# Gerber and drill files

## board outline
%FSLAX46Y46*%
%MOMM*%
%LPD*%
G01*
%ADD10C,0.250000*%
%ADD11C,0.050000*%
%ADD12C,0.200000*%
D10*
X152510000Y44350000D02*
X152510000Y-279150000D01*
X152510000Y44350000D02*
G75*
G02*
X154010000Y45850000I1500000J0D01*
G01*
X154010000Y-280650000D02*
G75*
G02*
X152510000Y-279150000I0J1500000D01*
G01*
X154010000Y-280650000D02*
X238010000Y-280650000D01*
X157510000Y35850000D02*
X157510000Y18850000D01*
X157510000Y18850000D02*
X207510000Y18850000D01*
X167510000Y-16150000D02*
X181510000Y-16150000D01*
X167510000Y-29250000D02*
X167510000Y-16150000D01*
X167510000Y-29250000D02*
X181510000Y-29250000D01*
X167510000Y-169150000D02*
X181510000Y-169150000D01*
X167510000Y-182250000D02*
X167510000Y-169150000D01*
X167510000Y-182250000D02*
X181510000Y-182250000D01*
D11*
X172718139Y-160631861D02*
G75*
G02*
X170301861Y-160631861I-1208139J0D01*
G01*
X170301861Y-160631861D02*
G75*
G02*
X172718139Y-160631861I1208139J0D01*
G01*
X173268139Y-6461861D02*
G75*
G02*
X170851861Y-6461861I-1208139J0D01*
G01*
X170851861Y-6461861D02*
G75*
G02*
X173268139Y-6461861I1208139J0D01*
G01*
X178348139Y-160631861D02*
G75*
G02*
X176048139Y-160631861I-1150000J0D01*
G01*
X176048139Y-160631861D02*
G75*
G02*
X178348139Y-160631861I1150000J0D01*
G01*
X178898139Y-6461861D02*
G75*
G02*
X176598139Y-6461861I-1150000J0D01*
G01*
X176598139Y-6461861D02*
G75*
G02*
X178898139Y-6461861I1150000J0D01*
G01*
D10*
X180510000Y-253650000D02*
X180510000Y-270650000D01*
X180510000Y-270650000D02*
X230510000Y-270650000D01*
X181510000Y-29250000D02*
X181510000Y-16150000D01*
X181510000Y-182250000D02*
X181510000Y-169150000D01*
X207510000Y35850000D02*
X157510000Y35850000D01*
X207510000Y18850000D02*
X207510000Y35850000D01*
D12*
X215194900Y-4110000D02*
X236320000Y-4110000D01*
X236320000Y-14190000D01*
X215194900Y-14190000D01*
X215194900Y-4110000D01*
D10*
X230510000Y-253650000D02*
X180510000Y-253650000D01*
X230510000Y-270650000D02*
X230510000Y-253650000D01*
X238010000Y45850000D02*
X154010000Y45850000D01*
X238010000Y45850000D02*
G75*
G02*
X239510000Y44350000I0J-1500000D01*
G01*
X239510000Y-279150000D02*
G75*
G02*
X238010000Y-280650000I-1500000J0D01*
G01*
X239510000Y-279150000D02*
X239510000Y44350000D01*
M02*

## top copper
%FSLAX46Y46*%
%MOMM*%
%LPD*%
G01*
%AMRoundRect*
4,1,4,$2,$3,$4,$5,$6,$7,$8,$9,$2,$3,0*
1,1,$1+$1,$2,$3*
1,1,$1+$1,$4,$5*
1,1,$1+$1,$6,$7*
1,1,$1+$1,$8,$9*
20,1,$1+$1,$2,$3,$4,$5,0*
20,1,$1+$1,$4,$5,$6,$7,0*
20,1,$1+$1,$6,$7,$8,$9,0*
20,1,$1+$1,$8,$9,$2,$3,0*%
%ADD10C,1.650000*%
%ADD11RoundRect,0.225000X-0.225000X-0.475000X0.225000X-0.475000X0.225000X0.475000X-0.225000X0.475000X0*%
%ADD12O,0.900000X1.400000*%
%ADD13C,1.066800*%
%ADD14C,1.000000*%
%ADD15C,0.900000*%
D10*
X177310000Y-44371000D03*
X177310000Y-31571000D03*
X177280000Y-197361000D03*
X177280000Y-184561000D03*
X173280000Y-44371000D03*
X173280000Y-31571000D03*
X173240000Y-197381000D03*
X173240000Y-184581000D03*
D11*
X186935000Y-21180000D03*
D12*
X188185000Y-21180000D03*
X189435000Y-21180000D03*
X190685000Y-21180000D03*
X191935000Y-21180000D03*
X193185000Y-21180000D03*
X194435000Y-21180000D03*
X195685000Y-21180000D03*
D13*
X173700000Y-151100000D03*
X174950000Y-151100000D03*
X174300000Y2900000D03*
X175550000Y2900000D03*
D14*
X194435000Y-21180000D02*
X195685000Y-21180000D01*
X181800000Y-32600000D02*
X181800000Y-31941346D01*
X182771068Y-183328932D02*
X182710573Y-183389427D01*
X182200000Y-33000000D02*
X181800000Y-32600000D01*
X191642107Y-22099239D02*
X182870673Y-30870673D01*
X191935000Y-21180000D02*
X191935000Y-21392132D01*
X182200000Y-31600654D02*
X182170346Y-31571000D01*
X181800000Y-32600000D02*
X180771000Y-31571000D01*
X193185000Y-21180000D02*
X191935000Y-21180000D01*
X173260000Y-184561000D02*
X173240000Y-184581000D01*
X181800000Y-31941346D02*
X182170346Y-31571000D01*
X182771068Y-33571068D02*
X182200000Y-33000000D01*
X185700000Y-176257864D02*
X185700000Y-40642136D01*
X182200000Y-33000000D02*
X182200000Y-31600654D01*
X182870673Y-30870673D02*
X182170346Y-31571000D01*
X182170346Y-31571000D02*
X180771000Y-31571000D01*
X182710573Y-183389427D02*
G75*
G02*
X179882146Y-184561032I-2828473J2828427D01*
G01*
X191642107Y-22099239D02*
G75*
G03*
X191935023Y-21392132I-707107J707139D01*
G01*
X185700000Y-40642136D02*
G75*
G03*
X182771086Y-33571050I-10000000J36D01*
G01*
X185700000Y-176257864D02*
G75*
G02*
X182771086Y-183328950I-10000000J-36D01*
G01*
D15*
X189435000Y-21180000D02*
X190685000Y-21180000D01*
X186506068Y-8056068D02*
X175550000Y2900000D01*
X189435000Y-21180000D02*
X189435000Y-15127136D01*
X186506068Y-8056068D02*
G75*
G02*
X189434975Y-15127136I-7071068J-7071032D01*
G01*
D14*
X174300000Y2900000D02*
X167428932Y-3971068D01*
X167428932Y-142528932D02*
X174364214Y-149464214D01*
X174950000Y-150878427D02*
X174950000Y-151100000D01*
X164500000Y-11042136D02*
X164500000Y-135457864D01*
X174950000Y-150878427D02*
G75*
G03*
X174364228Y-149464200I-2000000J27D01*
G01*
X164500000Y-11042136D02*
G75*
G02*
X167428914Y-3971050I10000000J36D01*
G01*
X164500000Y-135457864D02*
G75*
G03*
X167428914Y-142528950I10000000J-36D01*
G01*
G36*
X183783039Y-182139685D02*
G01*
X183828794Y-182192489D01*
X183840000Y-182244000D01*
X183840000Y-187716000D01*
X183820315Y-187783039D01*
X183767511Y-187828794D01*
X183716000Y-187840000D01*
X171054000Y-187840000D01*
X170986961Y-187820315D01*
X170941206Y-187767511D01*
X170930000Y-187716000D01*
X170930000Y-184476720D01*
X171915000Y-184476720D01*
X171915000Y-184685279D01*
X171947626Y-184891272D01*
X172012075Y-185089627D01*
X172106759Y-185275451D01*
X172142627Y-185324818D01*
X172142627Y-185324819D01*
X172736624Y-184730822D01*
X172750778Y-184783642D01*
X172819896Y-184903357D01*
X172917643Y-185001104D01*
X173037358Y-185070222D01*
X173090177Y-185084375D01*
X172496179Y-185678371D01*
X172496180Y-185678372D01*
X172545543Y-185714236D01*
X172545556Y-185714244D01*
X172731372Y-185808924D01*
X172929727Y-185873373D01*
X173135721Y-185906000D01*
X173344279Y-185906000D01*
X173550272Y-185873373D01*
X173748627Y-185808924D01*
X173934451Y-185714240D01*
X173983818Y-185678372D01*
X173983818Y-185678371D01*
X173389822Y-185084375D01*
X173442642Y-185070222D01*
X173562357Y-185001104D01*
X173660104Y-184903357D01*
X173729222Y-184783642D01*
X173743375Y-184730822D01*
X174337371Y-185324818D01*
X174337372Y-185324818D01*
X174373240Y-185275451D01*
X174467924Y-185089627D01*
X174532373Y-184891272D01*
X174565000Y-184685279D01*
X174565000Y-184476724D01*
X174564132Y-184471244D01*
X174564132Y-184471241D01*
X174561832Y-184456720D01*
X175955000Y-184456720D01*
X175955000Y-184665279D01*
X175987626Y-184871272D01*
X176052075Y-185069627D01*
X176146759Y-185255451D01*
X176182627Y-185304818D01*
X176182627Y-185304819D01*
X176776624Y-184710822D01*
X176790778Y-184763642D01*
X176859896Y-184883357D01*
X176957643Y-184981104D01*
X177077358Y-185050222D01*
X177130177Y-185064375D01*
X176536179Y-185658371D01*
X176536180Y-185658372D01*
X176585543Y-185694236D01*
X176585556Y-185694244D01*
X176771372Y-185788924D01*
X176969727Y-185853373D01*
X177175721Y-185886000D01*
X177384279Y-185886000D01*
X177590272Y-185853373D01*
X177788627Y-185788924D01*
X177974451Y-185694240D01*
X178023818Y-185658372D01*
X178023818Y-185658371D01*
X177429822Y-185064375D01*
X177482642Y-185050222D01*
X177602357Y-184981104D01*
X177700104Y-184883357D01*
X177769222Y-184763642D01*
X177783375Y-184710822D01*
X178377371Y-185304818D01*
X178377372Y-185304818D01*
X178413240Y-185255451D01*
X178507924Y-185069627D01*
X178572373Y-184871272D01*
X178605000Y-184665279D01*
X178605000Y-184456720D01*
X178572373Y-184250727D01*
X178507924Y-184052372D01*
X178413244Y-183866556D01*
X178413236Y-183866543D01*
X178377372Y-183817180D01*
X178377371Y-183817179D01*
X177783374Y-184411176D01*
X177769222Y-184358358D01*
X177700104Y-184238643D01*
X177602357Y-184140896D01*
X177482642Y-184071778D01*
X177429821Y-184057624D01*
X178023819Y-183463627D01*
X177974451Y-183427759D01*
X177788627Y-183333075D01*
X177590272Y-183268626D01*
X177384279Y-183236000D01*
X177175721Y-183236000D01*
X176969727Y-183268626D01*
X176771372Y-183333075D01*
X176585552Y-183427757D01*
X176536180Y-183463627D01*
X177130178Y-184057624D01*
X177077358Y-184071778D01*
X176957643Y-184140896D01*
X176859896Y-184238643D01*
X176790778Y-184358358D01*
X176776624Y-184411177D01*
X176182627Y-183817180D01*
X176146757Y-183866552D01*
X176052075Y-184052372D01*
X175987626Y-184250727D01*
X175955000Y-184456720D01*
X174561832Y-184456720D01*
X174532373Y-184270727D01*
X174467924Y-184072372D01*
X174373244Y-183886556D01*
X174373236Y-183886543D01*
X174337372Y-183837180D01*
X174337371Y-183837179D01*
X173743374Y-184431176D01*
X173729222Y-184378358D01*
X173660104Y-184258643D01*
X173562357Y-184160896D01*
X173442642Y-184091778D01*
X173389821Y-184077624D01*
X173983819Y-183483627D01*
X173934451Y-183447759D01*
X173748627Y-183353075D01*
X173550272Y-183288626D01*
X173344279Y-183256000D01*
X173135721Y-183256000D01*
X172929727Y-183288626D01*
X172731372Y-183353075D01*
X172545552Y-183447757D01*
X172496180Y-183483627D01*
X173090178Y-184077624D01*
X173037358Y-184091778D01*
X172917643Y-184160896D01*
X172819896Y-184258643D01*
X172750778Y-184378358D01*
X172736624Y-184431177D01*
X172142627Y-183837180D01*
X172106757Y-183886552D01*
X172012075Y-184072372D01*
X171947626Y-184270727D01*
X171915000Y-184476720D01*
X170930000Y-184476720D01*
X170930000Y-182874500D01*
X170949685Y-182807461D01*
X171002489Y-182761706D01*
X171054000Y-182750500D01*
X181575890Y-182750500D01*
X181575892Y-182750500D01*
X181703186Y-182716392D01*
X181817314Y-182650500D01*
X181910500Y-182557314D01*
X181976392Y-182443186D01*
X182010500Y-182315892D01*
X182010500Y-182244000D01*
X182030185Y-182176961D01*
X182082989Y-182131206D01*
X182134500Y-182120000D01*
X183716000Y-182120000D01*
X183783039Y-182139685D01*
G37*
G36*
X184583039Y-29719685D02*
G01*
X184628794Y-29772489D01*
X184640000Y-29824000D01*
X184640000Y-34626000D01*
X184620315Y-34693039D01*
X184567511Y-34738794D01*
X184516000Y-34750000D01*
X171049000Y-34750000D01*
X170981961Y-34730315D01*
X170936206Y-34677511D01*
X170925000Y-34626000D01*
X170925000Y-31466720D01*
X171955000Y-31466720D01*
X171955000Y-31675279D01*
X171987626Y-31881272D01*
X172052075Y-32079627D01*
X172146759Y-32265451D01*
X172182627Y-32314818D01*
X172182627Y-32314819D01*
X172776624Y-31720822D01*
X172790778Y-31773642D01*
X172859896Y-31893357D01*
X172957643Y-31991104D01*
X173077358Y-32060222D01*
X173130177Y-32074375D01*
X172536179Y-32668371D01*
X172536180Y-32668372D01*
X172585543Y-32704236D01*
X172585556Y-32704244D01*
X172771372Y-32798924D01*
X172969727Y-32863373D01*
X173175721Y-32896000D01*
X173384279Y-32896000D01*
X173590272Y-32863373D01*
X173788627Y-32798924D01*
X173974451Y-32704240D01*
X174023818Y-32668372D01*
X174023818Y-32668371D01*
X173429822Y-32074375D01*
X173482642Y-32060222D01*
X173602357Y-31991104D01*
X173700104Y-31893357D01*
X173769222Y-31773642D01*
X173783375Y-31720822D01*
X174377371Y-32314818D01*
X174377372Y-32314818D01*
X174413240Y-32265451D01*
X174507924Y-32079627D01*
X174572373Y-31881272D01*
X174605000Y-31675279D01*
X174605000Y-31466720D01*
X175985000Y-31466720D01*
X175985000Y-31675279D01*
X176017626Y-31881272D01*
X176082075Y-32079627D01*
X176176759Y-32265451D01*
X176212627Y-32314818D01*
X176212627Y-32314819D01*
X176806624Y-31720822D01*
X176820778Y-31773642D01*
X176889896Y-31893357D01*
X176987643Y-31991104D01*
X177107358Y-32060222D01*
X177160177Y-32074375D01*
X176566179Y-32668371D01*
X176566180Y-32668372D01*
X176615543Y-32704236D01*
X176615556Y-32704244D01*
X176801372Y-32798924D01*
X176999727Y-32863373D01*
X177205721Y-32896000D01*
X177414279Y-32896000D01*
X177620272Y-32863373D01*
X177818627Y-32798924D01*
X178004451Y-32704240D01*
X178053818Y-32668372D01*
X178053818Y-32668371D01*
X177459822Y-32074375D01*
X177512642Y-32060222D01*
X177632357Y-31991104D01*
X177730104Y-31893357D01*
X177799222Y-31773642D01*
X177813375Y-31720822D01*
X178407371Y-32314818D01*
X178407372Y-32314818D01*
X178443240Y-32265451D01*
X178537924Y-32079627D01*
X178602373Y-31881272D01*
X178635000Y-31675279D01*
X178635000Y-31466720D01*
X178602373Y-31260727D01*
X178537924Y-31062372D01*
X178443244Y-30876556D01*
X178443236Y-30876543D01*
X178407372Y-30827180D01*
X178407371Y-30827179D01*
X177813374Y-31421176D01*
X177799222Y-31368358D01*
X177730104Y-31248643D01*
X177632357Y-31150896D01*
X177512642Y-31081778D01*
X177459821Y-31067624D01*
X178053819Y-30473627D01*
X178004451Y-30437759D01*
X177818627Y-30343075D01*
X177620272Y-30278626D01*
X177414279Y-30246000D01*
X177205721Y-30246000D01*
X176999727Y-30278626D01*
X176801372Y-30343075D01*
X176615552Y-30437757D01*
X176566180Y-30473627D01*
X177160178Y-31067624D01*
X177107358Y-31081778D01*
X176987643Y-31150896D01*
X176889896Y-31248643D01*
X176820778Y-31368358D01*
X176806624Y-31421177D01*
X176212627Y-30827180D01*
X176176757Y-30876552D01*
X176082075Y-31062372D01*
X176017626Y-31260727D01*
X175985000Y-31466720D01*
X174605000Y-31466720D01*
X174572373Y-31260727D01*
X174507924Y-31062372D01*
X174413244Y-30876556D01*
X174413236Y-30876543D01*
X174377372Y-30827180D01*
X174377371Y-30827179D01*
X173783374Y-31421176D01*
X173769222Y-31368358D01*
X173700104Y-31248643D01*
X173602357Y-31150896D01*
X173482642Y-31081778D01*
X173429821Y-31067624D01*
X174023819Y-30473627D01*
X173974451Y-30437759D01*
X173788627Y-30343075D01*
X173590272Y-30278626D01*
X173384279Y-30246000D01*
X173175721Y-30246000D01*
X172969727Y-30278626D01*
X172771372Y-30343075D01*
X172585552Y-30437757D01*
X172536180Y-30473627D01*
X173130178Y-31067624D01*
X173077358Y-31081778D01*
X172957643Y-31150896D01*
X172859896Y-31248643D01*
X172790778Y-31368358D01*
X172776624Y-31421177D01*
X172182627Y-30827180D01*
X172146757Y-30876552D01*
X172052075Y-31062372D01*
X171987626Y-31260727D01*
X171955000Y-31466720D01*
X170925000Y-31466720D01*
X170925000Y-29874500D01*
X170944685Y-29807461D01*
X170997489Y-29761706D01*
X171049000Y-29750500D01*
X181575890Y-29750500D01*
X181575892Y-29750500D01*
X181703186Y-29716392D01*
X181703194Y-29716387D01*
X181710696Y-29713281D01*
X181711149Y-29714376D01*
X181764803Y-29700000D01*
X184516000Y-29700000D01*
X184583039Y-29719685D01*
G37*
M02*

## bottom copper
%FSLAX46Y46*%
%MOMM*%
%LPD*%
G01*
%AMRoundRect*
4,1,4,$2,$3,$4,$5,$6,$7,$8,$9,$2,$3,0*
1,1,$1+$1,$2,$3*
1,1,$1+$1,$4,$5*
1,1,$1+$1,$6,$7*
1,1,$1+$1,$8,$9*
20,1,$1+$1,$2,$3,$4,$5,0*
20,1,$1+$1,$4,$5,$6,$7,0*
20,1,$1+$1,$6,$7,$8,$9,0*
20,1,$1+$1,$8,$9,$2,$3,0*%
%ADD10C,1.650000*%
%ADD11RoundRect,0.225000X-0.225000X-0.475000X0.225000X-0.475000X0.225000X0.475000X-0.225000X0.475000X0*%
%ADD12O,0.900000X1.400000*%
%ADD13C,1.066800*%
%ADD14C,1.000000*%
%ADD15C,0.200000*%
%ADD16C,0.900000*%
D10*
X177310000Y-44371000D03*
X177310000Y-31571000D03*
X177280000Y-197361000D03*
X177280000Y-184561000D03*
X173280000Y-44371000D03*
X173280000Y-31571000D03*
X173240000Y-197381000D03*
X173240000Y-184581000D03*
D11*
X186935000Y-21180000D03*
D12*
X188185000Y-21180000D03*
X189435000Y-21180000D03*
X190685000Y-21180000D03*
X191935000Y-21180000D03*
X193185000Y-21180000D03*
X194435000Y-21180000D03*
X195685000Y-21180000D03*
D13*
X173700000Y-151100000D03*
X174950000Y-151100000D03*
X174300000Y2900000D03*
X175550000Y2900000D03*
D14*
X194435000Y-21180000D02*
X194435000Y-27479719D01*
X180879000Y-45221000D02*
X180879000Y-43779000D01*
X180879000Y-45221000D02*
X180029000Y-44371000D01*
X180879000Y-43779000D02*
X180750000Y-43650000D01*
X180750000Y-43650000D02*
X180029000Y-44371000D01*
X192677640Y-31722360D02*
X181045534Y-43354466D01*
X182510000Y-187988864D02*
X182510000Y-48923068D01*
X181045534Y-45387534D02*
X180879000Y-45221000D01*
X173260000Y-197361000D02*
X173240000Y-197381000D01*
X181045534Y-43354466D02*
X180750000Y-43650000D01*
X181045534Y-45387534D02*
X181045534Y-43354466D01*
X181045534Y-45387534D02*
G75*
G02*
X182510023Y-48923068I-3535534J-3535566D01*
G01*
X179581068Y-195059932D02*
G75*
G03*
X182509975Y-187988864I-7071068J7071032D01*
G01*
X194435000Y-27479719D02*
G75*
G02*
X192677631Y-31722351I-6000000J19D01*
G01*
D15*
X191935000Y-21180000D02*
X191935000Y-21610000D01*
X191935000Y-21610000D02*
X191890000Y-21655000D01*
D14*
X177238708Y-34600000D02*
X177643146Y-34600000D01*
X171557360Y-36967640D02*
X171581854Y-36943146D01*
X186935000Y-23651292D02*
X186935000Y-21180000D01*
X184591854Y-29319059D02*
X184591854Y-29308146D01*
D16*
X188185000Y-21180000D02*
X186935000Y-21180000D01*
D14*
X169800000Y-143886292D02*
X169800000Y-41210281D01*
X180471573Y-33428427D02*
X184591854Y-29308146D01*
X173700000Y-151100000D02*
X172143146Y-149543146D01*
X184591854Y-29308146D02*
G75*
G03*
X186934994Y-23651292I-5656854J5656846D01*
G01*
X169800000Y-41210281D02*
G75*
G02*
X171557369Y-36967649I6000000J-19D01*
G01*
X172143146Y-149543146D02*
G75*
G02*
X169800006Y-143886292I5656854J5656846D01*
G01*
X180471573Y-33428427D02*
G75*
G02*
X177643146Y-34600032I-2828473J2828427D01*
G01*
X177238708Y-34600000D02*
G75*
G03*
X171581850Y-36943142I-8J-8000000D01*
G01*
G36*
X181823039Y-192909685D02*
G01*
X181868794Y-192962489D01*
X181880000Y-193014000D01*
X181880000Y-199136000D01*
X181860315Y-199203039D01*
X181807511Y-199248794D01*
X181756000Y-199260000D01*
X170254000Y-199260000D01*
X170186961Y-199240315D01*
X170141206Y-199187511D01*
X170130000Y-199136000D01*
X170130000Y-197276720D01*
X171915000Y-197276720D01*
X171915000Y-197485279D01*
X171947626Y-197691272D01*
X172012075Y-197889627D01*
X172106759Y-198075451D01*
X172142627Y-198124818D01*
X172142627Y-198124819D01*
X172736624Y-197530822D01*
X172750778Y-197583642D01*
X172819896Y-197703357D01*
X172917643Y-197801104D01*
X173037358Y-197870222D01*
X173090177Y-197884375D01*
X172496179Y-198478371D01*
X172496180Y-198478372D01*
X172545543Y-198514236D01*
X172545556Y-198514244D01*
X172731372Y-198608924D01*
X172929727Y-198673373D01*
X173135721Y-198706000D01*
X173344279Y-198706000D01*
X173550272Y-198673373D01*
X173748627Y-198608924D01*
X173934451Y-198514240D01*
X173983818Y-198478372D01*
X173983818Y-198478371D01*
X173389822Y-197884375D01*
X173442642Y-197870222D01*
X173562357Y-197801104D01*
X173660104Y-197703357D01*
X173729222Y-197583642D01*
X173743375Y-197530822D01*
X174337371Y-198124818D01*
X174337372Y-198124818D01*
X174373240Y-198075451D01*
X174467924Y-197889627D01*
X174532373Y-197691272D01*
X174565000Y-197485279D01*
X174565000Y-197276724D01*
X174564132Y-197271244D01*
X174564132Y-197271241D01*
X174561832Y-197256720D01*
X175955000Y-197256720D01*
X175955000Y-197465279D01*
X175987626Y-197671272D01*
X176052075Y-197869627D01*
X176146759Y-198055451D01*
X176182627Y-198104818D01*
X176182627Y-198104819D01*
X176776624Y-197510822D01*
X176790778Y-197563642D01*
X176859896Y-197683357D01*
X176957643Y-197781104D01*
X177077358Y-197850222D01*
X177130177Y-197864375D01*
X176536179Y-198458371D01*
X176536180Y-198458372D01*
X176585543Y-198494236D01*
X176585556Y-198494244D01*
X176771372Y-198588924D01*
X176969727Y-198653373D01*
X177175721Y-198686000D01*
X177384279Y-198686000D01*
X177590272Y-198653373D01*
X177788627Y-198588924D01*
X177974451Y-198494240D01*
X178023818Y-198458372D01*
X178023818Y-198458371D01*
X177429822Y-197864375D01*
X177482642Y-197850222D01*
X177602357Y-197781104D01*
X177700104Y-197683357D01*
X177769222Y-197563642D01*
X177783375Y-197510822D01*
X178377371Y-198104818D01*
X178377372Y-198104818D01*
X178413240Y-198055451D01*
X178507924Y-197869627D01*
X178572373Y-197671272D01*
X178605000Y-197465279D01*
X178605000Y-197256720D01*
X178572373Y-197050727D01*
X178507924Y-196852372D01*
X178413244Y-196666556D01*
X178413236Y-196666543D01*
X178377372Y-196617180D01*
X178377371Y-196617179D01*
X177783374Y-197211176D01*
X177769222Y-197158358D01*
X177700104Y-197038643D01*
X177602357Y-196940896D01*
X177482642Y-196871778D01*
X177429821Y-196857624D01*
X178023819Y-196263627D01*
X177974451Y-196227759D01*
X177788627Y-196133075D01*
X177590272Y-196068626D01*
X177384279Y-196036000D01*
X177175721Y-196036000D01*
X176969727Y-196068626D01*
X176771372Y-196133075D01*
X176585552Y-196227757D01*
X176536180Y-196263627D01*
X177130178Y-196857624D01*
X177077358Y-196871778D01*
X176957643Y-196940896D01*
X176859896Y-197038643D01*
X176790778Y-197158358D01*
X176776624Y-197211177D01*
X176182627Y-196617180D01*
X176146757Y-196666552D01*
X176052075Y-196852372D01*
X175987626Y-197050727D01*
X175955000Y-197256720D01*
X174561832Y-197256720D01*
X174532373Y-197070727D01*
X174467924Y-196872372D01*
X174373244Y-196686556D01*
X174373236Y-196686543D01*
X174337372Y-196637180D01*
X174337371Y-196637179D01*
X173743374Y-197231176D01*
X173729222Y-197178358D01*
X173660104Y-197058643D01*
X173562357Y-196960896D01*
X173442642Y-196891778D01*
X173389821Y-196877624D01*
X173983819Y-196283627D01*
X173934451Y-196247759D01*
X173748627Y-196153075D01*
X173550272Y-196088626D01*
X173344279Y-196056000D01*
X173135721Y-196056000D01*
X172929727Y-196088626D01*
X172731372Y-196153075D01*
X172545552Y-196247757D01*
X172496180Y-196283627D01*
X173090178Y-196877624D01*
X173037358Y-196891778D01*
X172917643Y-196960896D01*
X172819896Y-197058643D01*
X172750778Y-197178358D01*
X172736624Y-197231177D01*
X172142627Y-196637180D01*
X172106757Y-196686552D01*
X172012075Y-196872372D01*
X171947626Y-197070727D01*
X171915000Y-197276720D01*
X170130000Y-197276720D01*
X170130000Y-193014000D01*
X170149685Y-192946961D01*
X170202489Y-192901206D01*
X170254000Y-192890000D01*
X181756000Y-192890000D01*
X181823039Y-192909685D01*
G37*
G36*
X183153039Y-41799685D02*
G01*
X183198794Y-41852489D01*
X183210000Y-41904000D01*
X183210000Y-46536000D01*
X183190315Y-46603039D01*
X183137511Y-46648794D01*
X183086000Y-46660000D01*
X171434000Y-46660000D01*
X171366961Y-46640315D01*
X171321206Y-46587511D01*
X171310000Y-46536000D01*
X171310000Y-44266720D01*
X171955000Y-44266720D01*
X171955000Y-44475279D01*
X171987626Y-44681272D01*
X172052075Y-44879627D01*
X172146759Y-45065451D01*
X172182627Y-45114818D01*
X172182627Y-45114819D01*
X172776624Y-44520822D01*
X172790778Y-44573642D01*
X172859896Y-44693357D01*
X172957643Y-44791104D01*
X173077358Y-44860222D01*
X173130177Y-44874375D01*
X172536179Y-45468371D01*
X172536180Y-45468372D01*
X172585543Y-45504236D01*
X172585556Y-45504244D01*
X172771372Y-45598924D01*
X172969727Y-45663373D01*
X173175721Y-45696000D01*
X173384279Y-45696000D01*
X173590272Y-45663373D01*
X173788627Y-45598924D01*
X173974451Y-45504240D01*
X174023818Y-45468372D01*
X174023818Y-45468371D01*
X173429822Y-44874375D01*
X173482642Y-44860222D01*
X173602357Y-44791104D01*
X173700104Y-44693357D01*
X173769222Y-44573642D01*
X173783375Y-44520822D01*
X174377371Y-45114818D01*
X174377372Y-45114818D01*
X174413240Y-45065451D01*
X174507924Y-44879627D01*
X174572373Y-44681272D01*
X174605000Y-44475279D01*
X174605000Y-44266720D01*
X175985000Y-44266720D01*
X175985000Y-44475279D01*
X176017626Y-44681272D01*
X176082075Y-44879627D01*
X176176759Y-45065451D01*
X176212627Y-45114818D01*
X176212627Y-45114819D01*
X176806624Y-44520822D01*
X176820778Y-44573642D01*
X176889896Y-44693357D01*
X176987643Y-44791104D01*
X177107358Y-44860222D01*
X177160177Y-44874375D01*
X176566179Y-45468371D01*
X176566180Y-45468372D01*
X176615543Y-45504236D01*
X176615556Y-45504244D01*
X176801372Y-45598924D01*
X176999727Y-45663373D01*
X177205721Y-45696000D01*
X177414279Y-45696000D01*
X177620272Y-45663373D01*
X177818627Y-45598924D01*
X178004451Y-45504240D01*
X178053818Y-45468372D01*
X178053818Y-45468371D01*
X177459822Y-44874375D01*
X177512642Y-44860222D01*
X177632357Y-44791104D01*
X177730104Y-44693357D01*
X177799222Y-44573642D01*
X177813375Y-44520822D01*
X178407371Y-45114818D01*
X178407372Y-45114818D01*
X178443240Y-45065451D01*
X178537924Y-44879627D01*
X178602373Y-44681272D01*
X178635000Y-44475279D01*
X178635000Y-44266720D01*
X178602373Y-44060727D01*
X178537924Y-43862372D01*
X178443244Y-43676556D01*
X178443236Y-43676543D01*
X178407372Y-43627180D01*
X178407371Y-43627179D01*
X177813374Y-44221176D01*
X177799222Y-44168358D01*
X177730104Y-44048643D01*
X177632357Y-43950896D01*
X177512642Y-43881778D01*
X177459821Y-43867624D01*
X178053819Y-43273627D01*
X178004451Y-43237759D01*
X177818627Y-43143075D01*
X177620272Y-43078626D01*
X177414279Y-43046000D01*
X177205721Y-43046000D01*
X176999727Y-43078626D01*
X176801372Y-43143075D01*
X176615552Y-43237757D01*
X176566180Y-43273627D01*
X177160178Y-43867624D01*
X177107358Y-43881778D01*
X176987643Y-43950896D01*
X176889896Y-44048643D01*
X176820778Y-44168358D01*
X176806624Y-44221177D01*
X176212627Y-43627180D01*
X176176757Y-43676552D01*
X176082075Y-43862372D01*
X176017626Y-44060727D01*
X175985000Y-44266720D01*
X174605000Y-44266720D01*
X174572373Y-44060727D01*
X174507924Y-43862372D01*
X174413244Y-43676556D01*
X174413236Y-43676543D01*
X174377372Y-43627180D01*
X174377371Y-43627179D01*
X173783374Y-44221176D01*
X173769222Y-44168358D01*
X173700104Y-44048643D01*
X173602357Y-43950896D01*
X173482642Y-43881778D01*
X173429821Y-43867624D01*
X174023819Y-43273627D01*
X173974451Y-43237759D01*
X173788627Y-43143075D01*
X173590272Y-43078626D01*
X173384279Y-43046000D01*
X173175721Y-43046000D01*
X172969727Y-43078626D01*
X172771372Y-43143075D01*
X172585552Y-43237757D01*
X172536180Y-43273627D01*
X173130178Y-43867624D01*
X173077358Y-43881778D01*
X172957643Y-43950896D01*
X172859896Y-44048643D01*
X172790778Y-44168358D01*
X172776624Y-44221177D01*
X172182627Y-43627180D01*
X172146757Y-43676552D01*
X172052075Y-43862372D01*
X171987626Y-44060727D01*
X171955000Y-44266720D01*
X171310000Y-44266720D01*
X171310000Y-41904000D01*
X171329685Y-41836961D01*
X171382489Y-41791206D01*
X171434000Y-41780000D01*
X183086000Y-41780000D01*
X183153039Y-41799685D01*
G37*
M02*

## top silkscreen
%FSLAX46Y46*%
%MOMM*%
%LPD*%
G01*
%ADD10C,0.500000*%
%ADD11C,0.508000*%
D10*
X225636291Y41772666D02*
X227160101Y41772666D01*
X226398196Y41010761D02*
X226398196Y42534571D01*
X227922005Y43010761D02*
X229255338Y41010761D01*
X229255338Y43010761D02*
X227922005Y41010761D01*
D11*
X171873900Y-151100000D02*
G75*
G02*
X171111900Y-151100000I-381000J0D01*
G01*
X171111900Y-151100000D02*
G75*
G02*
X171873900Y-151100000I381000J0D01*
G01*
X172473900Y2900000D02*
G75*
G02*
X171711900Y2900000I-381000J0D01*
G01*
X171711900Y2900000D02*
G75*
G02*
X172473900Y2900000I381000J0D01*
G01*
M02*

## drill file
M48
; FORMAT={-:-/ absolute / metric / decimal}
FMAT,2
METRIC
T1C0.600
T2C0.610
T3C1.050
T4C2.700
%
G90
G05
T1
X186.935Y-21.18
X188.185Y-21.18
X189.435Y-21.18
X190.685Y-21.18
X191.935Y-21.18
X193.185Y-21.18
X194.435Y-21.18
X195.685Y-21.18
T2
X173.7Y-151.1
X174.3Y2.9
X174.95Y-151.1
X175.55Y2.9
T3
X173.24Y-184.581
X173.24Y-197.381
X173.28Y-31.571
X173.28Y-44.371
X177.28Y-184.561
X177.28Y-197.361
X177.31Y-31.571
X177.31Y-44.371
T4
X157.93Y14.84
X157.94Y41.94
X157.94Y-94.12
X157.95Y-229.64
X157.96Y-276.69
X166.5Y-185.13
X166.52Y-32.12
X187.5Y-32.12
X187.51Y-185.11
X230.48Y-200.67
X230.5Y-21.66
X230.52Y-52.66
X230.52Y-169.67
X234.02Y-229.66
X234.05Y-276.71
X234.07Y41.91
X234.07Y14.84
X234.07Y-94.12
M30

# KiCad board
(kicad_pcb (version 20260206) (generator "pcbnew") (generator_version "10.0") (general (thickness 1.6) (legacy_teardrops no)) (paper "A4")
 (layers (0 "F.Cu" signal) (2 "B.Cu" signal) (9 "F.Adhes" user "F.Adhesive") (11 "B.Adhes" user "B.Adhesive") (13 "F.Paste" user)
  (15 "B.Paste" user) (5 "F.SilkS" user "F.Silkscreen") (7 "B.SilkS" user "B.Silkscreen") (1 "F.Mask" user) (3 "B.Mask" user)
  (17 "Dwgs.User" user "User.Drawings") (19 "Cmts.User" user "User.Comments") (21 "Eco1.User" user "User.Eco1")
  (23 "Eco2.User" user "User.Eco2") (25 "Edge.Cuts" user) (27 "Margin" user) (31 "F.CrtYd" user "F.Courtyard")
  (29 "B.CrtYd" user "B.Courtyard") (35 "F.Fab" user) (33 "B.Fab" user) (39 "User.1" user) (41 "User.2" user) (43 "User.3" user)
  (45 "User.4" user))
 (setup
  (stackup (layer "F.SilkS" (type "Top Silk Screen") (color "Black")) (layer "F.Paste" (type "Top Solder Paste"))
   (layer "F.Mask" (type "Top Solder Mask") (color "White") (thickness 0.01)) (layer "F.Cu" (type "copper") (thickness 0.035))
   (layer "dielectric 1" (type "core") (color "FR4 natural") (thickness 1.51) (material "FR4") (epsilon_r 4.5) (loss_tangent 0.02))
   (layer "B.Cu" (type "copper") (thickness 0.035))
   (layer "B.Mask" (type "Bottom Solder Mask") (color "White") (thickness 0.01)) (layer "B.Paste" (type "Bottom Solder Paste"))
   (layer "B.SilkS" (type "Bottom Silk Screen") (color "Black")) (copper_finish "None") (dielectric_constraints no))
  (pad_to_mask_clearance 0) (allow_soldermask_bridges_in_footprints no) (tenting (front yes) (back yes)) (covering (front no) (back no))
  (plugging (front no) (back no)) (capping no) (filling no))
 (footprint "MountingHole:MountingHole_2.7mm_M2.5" (layer "F.Cu") (at 230.52 169.67 180)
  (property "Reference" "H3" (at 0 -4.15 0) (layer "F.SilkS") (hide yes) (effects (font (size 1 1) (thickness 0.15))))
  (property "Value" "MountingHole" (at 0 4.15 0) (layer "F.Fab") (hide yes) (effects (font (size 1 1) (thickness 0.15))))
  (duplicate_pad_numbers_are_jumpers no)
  (pad "" np_thru_hole circle (at 0 0 180) (size 2.7 2.7) (drill 2.7) (layers "*.Cu" "*.Mask")))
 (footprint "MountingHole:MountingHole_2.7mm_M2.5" (layer "F.Cu") (at 187.5 32.12)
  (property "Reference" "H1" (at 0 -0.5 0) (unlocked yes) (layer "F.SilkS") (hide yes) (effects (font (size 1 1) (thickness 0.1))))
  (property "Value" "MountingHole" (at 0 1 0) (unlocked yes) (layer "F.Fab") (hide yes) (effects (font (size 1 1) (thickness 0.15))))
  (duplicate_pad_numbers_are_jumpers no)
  (pad "" np_thru_hole circle (at 0 0) (size 2.7 2.7) (drill 2.7) (layers "*.Cu" "*.Mask")))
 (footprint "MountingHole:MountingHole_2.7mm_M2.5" (layer "F.Cu") (at 234.07 -41.91 180)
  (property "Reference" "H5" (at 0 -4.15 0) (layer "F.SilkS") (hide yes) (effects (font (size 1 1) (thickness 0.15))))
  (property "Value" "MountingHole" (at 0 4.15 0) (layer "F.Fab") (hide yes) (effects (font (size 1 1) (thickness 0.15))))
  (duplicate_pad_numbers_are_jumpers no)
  (pad "" np_thru_hole circle (at 0 0 180) (size 2.7 2.7) (drill 2.7) (layers "*.Cu" "*.Mask")))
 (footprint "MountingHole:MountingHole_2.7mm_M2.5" (layer "F.Cu") (at 230.48 200.67 180)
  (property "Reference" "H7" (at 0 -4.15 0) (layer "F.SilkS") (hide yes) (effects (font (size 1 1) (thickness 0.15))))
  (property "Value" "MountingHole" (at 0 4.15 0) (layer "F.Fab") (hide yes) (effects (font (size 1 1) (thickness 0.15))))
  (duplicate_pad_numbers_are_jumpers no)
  (pad "" np_thru_hole circle (at 0 0 180) (size 2.7 2.7) (drill 2.7) (layers "*.Cu" "*.Mask")))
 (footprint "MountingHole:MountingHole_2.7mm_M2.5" (layer "F.Cu") (at 157.94 -41.94 180)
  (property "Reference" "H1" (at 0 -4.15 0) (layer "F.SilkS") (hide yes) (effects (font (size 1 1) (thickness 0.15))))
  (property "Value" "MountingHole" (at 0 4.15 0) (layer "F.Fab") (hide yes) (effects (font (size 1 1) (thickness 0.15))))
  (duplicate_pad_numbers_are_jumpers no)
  (pad "" np_thru_hole circle (at 0 0 180) (size 2.7 2.7) (drill 2.7) (layers "*.Cu" "*.Mask")))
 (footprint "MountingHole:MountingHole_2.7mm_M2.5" (layer "F.Cu") (at 166.5 185.13)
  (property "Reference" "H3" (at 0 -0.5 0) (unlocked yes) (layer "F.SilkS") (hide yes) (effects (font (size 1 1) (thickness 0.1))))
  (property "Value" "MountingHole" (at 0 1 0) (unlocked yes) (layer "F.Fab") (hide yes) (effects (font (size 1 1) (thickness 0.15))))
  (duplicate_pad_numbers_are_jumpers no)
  (pad "" np_thru_hole circle (at 0 0) (size 2.7 2.7) (drill 2.7) (layers "*.Cu" "*.Mask")))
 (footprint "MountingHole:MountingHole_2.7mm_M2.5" (layer "F.Cu") (at 234.05 276.71 180)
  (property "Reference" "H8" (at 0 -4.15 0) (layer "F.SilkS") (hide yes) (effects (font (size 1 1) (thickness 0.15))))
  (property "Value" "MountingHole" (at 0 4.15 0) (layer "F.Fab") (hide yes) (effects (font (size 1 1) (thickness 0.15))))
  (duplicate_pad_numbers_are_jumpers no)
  (pad "" np_thru_hole circle (at 0 0 180) (size 2.7 2.7) (drill 2.7) (layers "*.Cu" "*.Mask")))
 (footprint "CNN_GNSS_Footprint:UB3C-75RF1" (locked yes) (layer "F.Cu") (at 177.31 44.371 90)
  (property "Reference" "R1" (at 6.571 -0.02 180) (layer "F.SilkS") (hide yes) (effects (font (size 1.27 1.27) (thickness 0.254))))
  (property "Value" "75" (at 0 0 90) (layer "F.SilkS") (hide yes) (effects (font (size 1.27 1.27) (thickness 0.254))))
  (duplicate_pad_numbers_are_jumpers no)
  (pad "1" thru_hole circle (at 0 0 90) (size 1.65 1.65) (drill 1.05) (layers "*.Cu" "*.Mask") (remove_unused_layers no) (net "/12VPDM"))
  (pad "2" thru_hole circle (at 12.8 0 90) (size 1.65 1.65) (drill 1.05) (layers "*.Cu" "*.Mask") (remove_unused_layers no)
   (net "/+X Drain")))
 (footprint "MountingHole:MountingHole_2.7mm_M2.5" (layer "F.Cu") (at 230.52 52.66 180)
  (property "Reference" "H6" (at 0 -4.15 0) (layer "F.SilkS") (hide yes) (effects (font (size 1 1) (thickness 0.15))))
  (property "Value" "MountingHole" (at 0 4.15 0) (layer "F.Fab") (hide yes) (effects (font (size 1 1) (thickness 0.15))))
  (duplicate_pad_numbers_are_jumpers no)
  (pad "" np_thru_hole circle (at 0 0 180) (size 2.7 2.7) (drill 2.7) (layers "*.Cu" "*.Mask")))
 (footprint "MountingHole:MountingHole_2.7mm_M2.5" (layer "F.Cu") (at 166.52 32.12)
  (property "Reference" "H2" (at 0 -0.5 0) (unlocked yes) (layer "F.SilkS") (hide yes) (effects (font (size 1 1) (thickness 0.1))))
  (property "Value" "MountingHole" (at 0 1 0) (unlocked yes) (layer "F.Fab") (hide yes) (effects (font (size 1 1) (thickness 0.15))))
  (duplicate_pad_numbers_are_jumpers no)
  (pad "" np_thru_hole circle (at 0 0) (size 2.7 2.7) (drill 2.7) (layers "*.Cu" "*.Mask")))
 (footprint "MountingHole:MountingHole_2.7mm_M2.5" (layer "F.Cu") (at 234.07 -14.84 180)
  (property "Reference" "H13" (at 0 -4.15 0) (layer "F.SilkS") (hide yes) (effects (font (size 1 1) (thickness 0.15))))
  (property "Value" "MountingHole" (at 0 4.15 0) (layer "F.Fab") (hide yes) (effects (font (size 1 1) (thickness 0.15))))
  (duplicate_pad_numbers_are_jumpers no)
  (pad "" np_thru_hole circle (at 0 0 180) (size 2.7 2.7) (drill 2.7) (layers "*.Cu" "*.Mask")))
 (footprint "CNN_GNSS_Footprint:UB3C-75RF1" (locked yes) (layer "F.Cu") (at 177.28 197.361 90)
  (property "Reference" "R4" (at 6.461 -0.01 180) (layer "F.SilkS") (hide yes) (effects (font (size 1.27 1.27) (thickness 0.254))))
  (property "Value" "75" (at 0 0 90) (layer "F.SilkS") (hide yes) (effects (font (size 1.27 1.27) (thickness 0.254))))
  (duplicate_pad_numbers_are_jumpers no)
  (pad "1" thru_hole circle (at 0 0 90) (size 1.65 1.65) (drill 1.05) (layers "*.Cu" "*.Mask") (remove_unused_layers no) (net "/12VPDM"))
  (pad "2" thru_hole circle (at 12.8 0 90) (size 1.65 1.65) (drill 1.05) (layers "*.Cu" "*.Mask") (remove_unused_layers no)
   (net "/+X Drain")))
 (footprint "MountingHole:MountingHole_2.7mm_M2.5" (layer "F.Cu") (at 234.07 94.12 180)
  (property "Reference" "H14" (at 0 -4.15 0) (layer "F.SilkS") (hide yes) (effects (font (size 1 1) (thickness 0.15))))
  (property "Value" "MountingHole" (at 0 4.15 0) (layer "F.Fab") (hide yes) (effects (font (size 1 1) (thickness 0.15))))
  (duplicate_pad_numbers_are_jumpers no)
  (pad "" np_thru_hole circle (at 0 0 180) (size 2.7 2.7) (drill 2.7) (layers "*.Cu" "*.Mask")))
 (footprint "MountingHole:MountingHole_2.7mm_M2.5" (layer "F.Cu") (at 157.94 94.12 180)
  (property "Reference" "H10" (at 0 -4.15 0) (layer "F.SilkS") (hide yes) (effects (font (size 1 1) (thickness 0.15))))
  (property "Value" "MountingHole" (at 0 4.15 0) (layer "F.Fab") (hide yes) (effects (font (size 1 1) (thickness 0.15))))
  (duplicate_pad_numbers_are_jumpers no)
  (pad "" np_thru_hole circle (at 0 0 180) (size 2.7 2.7) (drill 2.7) (layers "*.Cu" "*.Mask")))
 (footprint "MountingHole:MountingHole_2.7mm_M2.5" (layer "F.Cu") (at 230.5 21.66 180)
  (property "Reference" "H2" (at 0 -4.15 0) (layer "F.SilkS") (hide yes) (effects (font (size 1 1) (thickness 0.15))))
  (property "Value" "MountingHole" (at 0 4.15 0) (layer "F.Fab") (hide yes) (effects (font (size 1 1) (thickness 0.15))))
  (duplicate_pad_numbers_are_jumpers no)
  (pad "" np_thru_hole circle (at 0 0 180) (size 2.7 2.7) (drill 2.7) (layers "*.Cu" "*.Mask")))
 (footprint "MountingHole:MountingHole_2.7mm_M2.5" (layer "F.Cu") (at 234.02 229.66 180)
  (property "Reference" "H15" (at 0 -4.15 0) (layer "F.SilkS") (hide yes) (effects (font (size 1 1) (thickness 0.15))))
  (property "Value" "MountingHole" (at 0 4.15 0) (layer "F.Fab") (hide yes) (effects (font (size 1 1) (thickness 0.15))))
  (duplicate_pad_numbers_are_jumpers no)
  (pad "" np_thru_hole circle (at 0 0 180) (size 2.7 2.7) (drill 2.7) (layers "*.Cu" "*.Mask")))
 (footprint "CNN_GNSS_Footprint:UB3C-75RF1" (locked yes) (layer "F.Cu") (at 173.28 44.371 90)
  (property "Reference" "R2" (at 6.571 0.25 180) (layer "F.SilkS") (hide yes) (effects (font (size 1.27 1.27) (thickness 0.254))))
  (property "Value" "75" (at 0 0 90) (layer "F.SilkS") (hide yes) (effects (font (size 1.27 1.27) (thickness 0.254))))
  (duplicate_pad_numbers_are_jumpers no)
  (pad "1" thru_hole circle (at 0 0 90) (size 1.65 1.65) (drill 1.05) (layers "*.Cu" "*.Mask") (remove_unused_layers no) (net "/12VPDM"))
  (pad "2" thru_hole circle (at 12.8 0 90) (size 1.65 1.65) (drill 1.05) (layers "*.Cu" "*.Mask") (remove_unused_layers no)
   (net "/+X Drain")))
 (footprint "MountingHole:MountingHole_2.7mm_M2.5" (layer "F.Cu") (at 157.95 229.64 180)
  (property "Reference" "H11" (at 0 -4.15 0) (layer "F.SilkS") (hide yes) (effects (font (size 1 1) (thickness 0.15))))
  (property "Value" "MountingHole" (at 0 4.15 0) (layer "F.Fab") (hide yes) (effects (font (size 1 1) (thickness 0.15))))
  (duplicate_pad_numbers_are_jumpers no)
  (pad "" np_thru_hole circle (at 0 0 180) (size 2.7 2.7) (drill 2.7) (layers "*.Cu" "*.Mask")))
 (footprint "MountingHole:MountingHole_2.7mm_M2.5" (layer "F.Cu") (at 157.93 -14.84 180)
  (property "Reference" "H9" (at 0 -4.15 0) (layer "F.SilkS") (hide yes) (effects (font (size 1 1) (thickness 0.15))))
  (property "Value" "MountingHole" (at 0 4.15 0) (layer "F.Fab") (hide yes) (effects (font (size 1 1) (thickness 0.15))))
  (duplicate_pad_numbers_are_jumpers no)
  (pad "" np_thru_hole circle (at 0 0 180) (size 2.7 2.7) (drill 2.7) (layers "*.Cu" "*.Mask")))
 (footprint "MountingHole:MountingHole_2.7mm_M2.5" (layer "F.Cu") (at 187.51 185.11)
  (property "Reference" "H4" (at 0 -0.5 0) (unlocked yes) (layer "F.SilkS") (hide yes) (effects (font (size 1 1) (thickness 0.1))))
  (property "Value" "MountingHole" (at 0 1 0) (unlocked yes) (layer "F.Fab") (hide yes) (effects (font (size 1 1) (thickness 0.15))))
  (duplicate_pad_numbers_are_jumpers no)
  (pad "" np_thru_hole circle (at 0 0) (size 2.7 2.7) (drill 2.7) (layers "*.Cu" "*.Mask")))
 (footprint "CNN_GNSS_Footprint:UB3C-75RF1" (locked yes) (layer "F.Cu") (at 173.24 197.381 90)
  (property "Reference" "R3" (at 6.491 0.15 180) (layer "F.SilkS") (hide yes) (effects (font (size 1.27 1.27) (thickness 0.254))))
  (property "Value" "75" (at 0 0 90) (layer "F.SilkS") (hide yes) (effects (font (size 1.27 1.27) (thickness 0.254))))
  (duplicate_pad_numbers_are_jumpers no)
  (pad "1" thru_hole circle (at 0 0 90) (size 1.65 1.65) (drill 1.05) (layers "*.Cu" "*.Mask") (remove_unused_layers no) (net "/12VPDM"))
  (pad "2" thru_hole circle (at 12.8 0 90) (size 1.65 1.65) (drill 1.05) (layers "*.Cu" "*.Mask") (remove_unused_layers no)
   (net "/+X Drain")))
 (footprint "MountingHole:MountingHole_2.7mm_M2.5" (layer "F.Cu") (at 157.96 276.69 180)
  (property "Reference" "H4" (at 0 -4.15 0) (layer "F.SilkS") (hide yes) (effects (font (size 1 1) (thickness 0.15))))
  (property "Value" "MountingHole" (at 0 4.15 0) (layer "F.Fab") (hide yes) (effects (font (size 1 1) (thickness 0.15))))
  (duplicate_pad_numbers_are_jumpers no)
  (pad "" np_thru_hole circle (at 0 0 180) (size 2.7 2.7) (drill 2.7) (layers "*.Cu" "*.Mask")))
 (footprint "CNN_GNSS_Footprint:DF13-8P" (layer "B.Cu") (at 190.98 21.73)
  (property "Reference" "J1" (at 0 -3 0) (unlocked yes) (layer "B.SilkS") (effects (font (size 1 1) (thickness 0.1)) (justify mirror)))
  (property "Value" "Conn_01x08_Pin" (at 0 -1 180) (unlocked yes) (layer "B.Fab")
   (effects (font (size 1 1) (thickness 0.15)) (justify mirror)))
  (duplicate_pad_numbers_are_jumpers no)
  (pad "1" thru_hole roundrect (at -4.045 -0.55) (size 0.9 1.4) (drill 0.6) (layers "*.Cu" "*.Mask") (remove_unused_layers no)
   (roundrect_rratio 0.25) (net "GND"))
  (pad "2" thru_hole oval (at -2.795 -0.55) (size 0.9 1.4) (drill 0.6) (layers "*.Cu" "*.Mask") (remove_unused_layers no) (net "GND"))
  (pad "3" thru_hole oval (at -1.545 -0.55) (size 0.9 1.4) (drill 0.6) (layers "*.Cu" "*.Mask") (remove_unused_layers no)
   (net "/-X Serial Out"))
  (pad "4" thru_hole oval (at -0.295 -0.55) (size 0.9 1.4) (drill 0.6) (layers "*.Cu" "*.Mask") (remove_unused_layers no)
   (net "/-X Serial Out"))
  (pad "5" thru_hole oval (at 0.955 -0.55) (size 0.9 1.4) (drill 0.6) (layers "*.Cu" "*.Mask") (remove_unused_layers no) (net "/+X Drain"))
  (pad "6" thru_hole oval (at 2.205 -0.55) (size 0.9 1.4) (drill 0.6) (layers "*.Cu" "*.Mask") (remove_unused_layers no) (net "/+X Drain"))
  (pad "7" thru_hole oval (at 3.455 -0.55) (size 0.9 1.4) (drill 0.6) (layers "*.Cu" "*.Mask") (remove_unused_layers no) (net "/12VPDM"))
  (pad "8" thru_hole oval (at 4.705 -0.55) (size 0.9 1.4) (drill 0.6) (layers "*.Cu" "*.Mask") (remove_unused_layers no) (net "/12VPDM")))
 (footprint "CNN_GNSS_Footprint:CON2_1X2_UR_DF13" (layer "B.Cu") (at 173.7 151.1 180)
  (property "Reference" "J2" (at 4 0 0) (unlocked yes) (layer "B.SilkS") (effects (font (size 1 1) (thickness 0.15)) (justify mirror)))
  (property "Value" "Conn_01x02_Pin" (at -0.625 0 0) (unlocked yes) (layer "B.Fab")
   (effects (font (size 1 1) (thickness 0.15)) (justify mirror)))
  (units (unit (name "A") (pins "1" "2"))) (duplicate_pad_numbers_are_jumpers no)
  (fp_circle (center 2.2071 0) (end 2.5881 0) (stroke (width 0.508) (type solid)) (fill no) (layer "F.SilkS"))
  (pad "1" thru_hole circle (at 0 0 180) (size 1.0668 1.0668) (drill 0.6096) (layers "*.Cu" "*.Mask") (remove_unused_layers no) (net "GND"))
  (pad "2" thru_hole circle (at -1.25 0 180) (size 1.0668 1.0668) (drill 0.6096) (layers "*.Cu" "*.Mask") (remove_unused_layers no)
   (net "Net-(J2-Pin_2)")))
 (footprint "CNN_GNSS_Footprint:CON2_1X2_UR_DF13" (layer "B.Cu") (at 174.3 -2.9 180)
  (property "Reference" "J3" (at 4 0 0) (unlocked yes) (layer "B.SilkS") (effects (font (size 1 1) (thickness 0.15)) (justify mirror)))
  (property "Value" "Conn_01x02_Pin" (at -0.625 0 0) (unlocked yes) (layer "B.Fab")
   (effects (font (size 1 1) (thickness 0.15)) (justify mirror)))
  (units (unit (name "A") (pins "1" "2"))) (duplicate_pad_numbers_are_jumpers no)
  (fp_circle (center 2.2071 0) (end 2.5881 0) (stroke (width 0.508) (type solid)) (fill no) (layer "F.SilkS"))
  (pad "1" thru_hole circle (at 0 0 180) (size 1.0668 1.0668) (drill 0.6096) (layers "*.Cu" "*.Mask") (remove_unused_layers no)
   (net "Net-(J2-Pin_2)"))
  (pad "2" thru_hole circle (at -1.25 0 180) (size 1.0668 1.0668) (drill 0.6096) (layers "*.Cu" "*.Mask") (remove_unused_layers no)
   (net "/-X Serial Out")))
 (gr_line (start 152.51 -44.35) (end 152.51 279.15) (stroke (width 0.25) (type default)) (layer "Edge.Cuts"))
 (gr_arc (start 152.51 -44.35) (mid 152.94934 -45.41066) (end 154.01 -45.85) (stroke (width 0.25) (type default)) (layer "Edge.Cuts"))
 (gr_arc (start 154.01 280.65) (mid 152.94934 280.21066) (end 152.51 279.15) (stroke (width 0.25) (type default)) (layer "Edge.Cuts"))
 (gr_line (start 154.01 280.65) (end 238.01 280.65) (stroke (width 0.25) (type default)) (layer "Edge.Cuts"))
 (gr_line (start 157.51 -35.85) (end 157.51 -18.85) (stroke (width 0.25) (type default)) (layer "Edge.Cuts"))
 (gr_line (start 157.51 -18.85) (end 207.51 -18.85) (stroke (width 0.25) (type default)) (layer "Edge.Cuts"))
 (gr_line (start 167.51 16.15) (end 181.51 16.15) (stroke (width 0.25) (type default)) (layer "Edge.Cuts"))
 (gr_line (start 167.51 29.25) (end 167.51 16.15) (stroke (width 0.25) (type default)) (layer "Edge.Cuts"))
 (gr_line (start 167.51 29.25) (end 181.51 29.25) (stroke (width 0.25) (type default)) (layer "Edge.Cuts"))
 (gr_line (start 167.51 169.15) (end 181.51 169.15) (stroke (width 0.25) (type default)) (layer "Edge.Cuts"))
 (gr_line (start 167.51 182.25) (end 167.51 169.15) (stroke (width 0.25) (type default)) (layer "Edge.Cuts"))
 (gr_line (start 167.51 182.25) (end 181.51 182.25) (stroke (width 0.25) (type default)) (layer "Edge.Cuts"))
 (gr_circle (center 171.51 160.631861) (end 171.91 161.771861) (stroke (width 0.05) (type default)) (fill no) (layer "Edge.Cuts"))
 (gr_circle (center 172.06 6.461861) (end 172.46 7.601861) (stroke (width 0.05) (type default)) (fill no) (layer "Edge.Cuts"))
 (gr_circle (center 177.198139 160.631861) (end 178.348139 160.631861) (stroke (width 0.05) (type solid)) (fill no) (layer "Edge.Cuts"))
 (gr_circle (center 177.748139 6.461861) (end 178.898139 6.461861) (stroke (width 0.05) (type solid)) (fill no) (layer "Edge.Cuts"))
 (gr_line (start 180.51 253.65) (end 180.51 270.65) (stroke (width 0.25) (type default)) (layer "Edge.Cuts"))
 (gr_line (start 180.51 270.65) (end 230.51 270.65) (stroke (width 0.25) (type default)) (layer "Edge.Cuts"))
 (gr_line (start 181.51 29.25) (end 181.51 16.15) (stroke (width 0.25) (type default)) (layer "Edge.Cuts"))
 (gr_line (start 181.51 182.25) (end 181.51 169.15) (stroke (width 0.25) (type default)) (layer "Edge.Cuts"))
 (gr_line (start 207.51 -35.85) (end 157.51 -35.85) (stroke (width 0.25) (type default)) (layer "Edge.Cuts"))
 (gr_line (start 207.51 -18.85) (end 207.51 -35.85) (stroke (width 0.25) (type default)) (layer "Edge.Cuts"))
 (gr_rect (start 215.1949 4.11) (end 236.32 14.19) (stroke (width 0.2) (type solid)) (fill no) (layer "Edge.Cuts"))
 (gr_line (start 230.51 253.65) (end 180.51 253.65) (stroke (width 0.25) (type default)) (layer "Edge.Cuts"))
 (gr_line (start 230.51 270.65) (end 230.51 253.65) (stroke (width 0.25) (type default)) (layer "Edge.Cuts"))
 (gr_line (start 238.01 -45.85) (end 154.01 -45.85) (stroke (width 0.25) (type default)) (layer "Edge.Cuts"))
 (gr_arc (start 238.01 -45.85) (mid 239.07066 -45.41066) (end 239.51 -44.35) (stroke (width 0.25) (type default)) (layer "Edge.Cuts"))
 (gr_arc (start 239.51 279.15) (mid 239.07066 280.21066) (end 238.01 280.65) (stroke (width 0.25) (type default)) (layer "Edge.Cuts"))
 (gr_line (start 239.51 279.15) (end 239.51 -44.35) (stroke (width 0.25) (type default)) (layer "Edge.Cuts"))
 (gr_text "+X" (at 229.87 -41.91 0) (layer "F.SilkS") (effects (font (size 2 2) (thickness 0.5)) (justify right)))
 (segment (start 194.435 21.18) (end 195.685 21.18) (width 1) (layer "F.Cu") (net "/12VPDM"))
 (segment (start 194.435 21.18) (end 194.435 27.479719) (width 1) (layer "B.Cu") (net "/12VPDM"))
 (segment (start 180.879 45.221) (end 180.879 43.779) (width 1) (layer "B.Cu") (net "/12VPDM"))
 (segment (start 180.879 45.221) (end 180.029 44.371) (width 1) (layer "B.Cu") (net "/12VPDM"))
 (segment (start 180.879 43.779) (end 180.75 43.65) (width 1) (layer "B.Cu") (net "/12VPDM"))
 (segment (start 180.75 43.65) (end 180.029 44.371) (width 1) (layer "B.Cu") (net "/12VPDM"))
 (segment (start 192.67764 31.72236) (end 181.045534 43.354466) (width 1) (layer "B.Cu") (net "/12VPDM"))
 (segment (start 182.51 187.988864) (end 182.51 48.923068) (width 1) (layer "B.Cu") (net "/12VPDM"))
 (segment (start 181.045534 45.387534) (end 180.879 45.221) (width 1) (layer "B.Cu") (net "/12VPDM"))
 (segment (start 173.26 197.361) (end 173.24 197.381) (width 1) (layer "B.Cu") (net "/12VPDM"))
 (segment (start 181.045534 43.354466) (end 180.75 43.65) (width 1) (layer "B.Cu") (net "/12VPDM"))
 (segment (start 181.045534 45.387534) (end 181.045534 43.354466) (width 1) (layer "B.Cu") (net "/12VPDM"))
 (arc (start 181.045534 45.387534) (mid 182.129398 47.009651) (end 182.51 48.923068) (width 1) (layer "B.Cu") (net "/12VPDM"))
 (arc (start 179.581068 195.059932) (mid 181.748796 191.815698) (end 182.51 187.988864) (width 1) (layer "B.Cu") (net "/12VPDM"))
 (arc (start 194.435 27.479719) (mid 193.978277 29.77582) (end 192.67764 31.72236) (width 1) (layer "B.Cu") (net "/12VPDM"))
 (segment (start 181.8 32.6) (end 181.8 31.941346) (width 1) (layer "F.Cu") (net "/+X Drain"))
 (segment (start 182.771068 183.328932) (end 182.710573 183.389427) (width 1) (layer "F.Cu") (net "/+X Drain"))
 (segment (start 182.2 33) (end 181.8 32.6) (width 1) (layer "F.Cu") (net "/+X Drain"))
 (segment (start 191.642107 22.099239) (end 182.870673 30.870673) (width 1) (layer "F.Cu") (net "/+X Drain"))
 (segment (start 191.935 21.18) (end 191.935 21.392132) (width 1) (layer "F.Cu") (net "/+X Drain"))
 (segment (start 182.2 31.600654) (end 182.170346 31.571) (width 1) (layer "F.Cu") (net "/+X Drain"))
 (segment (start 181.8 32.6) (end 180.771 31.571) (width 1) (layer "F.Cu") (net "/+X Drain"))
 (segment (start 193.185 21.18) (end 191.935 21.18) (width 1) (layer "F.Cu") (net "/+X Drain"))
 (segment (start 173.26 184.561) (end 173.24 184.581) (width 1) (layer "F.Cu") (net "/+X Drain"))
 (segment (start 181.8 31.941346) (end 182.170346 31.571) (width 1) (layer "F.Cu") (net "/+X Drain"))
 (segment (start 182.771068 33.571068) (end 182.2 33) (width 1) (layer "F.Cu") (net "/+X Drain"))
 (segment (start 185.7 176.257864) (end 185.7 40.642136) (width 1) (layer "F.Cu") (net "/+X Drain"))
 (segment (start 182.2 33) (end 182.2 31.600654) (width 1) (layer "F.Cu") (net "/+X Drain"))
 (segment (start 182.870673 30.870673) (end 182.170346 31.571) (width 1) (layer "F.Cu") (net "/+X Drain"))
 (segment (start 182.170346 31.571) (end 180.771 31.571) (width 1) (layer "F.Cu") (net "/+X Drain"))
 (arc (start 182.710573 183.389427) (mid 181.41288 184.256518) (end 179.882146 184.561) (width 1) (layer "F.Cu") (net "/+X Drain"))
 (arc (start 191.642107 22.099239) (mid 191.85888 21.774816) (end 191.935 21.392132) (width 1) (layer "F.Cu") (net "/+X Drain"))
 (arc (start 185.7 40.642136) (mid 184.938795 36.815302) (end 182.771068 33.571068) (width 1) (layer "F.Cu") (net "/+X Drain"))
 (arc (start 185.7 176.257864) (mid 184.938795 180.084698) (end 182.771068 183.328932) (width 1) (layer "F.Cu") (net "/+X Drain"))
 (segment (start 191.935 21.18) (end 191.935 21.61) (width 0.2) (layer "B.Cu") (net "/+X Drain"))
 (segment (start 191.935 21.61) (end 191.89 21.655) (width 0.2) (layer "B.Cu") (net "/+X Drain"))
 (segment (start 177.238708 34.6) (end 177.643146 34.6) (width 1) (layer "B.Cu") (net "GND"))
 (segment (start 171.55736 36.96764) (end 171.581854 36.943146) (width 1) (layer "B.Cu") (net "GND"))
 (segment (start 186.935 23.651292) (end 186.935 21.18) (width 1) (layer "B.Cu") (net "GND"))
 (segment (start 184.591854 29.319059) (end 184.591854 29.308146) (width 1) (layer "B.Cu") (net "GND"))
 (segment (start 188.185 21.18) (end 186.935 21.18) (width 0.9) (layer "B.Cu") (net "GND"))
 (segment (start 169.8 143.886292) (end 169.8 41.210281) (width 1) (layer "B.Cu") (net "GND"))
 (segment (start 180.471573 33.428427) (end 184.591854 29.308146) (width 1) (layer "B.Cu") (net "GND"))
 (segment (start 173.7 151.1) (end 172.143146 149.543146) (width 1) (layer "B.Cu") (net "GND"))
 (arc (start 184.591854 29.308146) (mid 186.326036 26.712759) (end 186.935 23.651292) (width 1) (layer "B.Cu") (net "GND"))
 (arc (start 169.8 41.210281) (mid 170.256723 38.91418) (end 171.55736 36.96764) (width 1) (layer "B.Cu") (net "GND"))
 (arc (start 172.143146 149.543146) (mid 170.408964 146.947759) (end 169.8 143.886292) (width 1) (layer "B.Cu") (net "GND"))
 (arc (start 180.471573 33.428427) (mid 179.17388 34.295518) (end 177.643146 34.6) (width 1) (layer "B.Cu") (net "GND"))
 (arc (start 177.238708 34.6) (mid 174.177241 35.208964) (end 171.581854 36.943146) (width 1) (layer "B.Cu") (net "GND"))
 (segment (start 189.435 21.18) (end 190.685 21.18) (width 0.9) (layer "F.Cu") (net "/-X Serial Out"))
 (segment (start 186.506068 8.056068) (end 175.55 -2.9) (width 0.9) (layer "F.Cu") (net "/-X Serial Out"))
 (segment (start 189.435 21.18) (end 189.435 15.127136) (width 0.9) (layer "F.Cu") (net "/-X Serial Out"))
 (arc (start 186.506068 8.056068) (mid 188.673796 11.300302) (end 189.435 15.127136) (width 0.9) (layer "F.Cu") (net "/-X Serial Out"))
 (segment (start 174.3 -2.9) (end 167.428932 3.971068) (width 1) (layer "F.Cu") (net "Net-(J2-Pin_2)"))
 (segment (start 167.428932 142.528932) (end 174.364214 149.464214) (width 1) (layer "F.Cu") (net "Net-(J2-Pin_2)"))
 (segment (start 174.95 150.878427) (end 174.95 151.1) (width 1) (layer "F.Cu") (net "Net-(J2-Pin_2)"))
 (segment (start 164.5 11.042136) (end 164.5 135.457864) (width 1) (layer "F.Cu") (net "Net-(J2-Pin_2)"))
 (arc (start 174.95 150.878427) (mid 174.797759 150.11306) (end 174.364214 149.464214) (width 1) (layer "F.Cu") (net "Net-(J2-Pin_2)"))
 (arc (start 164.5 11.042136) (mid 165.261205 7.215302) (end 167.428932 3.971068) (width 1) (layer "F.Cu") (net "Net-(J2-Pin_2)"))
 (arc (start 164.5 135.457864) (mid 165.261204 139.284698) (end 167.428932 142.528932) (width 1) (layer "F.Cu") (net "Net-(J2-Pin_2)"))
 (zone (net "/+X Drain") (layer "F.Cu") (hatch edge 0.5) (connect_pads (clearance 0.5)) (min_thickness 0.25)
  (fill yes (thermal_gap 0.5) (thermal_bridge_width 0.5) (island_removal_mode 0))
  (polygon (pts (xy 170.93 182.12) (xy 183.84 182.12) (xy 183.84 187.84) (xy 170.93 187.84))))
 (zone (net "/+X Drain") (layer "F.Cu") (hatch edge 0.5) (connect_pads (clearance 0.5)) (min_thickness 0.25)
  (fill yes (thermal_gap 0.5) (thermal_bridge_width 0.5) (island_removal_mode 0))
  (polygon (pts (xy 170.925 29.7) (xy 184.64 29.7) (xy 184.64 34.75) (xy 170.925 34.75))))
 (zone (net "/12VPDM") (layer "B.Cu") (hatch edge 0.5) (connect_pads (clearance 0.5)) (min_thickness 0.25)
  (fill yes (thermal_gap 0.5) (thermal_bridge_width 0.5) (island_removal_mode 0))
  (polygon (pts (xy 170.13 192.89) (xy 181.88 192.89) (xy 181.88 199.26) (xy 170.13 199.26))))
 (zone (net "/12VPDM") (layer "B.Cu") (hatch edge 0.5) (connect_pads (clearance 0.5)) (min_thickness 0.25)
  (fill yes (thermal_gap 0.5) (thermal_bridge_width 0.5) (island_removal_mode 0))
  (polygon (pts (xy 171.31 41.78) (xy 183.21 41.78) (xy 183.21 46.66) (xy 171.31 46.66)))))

